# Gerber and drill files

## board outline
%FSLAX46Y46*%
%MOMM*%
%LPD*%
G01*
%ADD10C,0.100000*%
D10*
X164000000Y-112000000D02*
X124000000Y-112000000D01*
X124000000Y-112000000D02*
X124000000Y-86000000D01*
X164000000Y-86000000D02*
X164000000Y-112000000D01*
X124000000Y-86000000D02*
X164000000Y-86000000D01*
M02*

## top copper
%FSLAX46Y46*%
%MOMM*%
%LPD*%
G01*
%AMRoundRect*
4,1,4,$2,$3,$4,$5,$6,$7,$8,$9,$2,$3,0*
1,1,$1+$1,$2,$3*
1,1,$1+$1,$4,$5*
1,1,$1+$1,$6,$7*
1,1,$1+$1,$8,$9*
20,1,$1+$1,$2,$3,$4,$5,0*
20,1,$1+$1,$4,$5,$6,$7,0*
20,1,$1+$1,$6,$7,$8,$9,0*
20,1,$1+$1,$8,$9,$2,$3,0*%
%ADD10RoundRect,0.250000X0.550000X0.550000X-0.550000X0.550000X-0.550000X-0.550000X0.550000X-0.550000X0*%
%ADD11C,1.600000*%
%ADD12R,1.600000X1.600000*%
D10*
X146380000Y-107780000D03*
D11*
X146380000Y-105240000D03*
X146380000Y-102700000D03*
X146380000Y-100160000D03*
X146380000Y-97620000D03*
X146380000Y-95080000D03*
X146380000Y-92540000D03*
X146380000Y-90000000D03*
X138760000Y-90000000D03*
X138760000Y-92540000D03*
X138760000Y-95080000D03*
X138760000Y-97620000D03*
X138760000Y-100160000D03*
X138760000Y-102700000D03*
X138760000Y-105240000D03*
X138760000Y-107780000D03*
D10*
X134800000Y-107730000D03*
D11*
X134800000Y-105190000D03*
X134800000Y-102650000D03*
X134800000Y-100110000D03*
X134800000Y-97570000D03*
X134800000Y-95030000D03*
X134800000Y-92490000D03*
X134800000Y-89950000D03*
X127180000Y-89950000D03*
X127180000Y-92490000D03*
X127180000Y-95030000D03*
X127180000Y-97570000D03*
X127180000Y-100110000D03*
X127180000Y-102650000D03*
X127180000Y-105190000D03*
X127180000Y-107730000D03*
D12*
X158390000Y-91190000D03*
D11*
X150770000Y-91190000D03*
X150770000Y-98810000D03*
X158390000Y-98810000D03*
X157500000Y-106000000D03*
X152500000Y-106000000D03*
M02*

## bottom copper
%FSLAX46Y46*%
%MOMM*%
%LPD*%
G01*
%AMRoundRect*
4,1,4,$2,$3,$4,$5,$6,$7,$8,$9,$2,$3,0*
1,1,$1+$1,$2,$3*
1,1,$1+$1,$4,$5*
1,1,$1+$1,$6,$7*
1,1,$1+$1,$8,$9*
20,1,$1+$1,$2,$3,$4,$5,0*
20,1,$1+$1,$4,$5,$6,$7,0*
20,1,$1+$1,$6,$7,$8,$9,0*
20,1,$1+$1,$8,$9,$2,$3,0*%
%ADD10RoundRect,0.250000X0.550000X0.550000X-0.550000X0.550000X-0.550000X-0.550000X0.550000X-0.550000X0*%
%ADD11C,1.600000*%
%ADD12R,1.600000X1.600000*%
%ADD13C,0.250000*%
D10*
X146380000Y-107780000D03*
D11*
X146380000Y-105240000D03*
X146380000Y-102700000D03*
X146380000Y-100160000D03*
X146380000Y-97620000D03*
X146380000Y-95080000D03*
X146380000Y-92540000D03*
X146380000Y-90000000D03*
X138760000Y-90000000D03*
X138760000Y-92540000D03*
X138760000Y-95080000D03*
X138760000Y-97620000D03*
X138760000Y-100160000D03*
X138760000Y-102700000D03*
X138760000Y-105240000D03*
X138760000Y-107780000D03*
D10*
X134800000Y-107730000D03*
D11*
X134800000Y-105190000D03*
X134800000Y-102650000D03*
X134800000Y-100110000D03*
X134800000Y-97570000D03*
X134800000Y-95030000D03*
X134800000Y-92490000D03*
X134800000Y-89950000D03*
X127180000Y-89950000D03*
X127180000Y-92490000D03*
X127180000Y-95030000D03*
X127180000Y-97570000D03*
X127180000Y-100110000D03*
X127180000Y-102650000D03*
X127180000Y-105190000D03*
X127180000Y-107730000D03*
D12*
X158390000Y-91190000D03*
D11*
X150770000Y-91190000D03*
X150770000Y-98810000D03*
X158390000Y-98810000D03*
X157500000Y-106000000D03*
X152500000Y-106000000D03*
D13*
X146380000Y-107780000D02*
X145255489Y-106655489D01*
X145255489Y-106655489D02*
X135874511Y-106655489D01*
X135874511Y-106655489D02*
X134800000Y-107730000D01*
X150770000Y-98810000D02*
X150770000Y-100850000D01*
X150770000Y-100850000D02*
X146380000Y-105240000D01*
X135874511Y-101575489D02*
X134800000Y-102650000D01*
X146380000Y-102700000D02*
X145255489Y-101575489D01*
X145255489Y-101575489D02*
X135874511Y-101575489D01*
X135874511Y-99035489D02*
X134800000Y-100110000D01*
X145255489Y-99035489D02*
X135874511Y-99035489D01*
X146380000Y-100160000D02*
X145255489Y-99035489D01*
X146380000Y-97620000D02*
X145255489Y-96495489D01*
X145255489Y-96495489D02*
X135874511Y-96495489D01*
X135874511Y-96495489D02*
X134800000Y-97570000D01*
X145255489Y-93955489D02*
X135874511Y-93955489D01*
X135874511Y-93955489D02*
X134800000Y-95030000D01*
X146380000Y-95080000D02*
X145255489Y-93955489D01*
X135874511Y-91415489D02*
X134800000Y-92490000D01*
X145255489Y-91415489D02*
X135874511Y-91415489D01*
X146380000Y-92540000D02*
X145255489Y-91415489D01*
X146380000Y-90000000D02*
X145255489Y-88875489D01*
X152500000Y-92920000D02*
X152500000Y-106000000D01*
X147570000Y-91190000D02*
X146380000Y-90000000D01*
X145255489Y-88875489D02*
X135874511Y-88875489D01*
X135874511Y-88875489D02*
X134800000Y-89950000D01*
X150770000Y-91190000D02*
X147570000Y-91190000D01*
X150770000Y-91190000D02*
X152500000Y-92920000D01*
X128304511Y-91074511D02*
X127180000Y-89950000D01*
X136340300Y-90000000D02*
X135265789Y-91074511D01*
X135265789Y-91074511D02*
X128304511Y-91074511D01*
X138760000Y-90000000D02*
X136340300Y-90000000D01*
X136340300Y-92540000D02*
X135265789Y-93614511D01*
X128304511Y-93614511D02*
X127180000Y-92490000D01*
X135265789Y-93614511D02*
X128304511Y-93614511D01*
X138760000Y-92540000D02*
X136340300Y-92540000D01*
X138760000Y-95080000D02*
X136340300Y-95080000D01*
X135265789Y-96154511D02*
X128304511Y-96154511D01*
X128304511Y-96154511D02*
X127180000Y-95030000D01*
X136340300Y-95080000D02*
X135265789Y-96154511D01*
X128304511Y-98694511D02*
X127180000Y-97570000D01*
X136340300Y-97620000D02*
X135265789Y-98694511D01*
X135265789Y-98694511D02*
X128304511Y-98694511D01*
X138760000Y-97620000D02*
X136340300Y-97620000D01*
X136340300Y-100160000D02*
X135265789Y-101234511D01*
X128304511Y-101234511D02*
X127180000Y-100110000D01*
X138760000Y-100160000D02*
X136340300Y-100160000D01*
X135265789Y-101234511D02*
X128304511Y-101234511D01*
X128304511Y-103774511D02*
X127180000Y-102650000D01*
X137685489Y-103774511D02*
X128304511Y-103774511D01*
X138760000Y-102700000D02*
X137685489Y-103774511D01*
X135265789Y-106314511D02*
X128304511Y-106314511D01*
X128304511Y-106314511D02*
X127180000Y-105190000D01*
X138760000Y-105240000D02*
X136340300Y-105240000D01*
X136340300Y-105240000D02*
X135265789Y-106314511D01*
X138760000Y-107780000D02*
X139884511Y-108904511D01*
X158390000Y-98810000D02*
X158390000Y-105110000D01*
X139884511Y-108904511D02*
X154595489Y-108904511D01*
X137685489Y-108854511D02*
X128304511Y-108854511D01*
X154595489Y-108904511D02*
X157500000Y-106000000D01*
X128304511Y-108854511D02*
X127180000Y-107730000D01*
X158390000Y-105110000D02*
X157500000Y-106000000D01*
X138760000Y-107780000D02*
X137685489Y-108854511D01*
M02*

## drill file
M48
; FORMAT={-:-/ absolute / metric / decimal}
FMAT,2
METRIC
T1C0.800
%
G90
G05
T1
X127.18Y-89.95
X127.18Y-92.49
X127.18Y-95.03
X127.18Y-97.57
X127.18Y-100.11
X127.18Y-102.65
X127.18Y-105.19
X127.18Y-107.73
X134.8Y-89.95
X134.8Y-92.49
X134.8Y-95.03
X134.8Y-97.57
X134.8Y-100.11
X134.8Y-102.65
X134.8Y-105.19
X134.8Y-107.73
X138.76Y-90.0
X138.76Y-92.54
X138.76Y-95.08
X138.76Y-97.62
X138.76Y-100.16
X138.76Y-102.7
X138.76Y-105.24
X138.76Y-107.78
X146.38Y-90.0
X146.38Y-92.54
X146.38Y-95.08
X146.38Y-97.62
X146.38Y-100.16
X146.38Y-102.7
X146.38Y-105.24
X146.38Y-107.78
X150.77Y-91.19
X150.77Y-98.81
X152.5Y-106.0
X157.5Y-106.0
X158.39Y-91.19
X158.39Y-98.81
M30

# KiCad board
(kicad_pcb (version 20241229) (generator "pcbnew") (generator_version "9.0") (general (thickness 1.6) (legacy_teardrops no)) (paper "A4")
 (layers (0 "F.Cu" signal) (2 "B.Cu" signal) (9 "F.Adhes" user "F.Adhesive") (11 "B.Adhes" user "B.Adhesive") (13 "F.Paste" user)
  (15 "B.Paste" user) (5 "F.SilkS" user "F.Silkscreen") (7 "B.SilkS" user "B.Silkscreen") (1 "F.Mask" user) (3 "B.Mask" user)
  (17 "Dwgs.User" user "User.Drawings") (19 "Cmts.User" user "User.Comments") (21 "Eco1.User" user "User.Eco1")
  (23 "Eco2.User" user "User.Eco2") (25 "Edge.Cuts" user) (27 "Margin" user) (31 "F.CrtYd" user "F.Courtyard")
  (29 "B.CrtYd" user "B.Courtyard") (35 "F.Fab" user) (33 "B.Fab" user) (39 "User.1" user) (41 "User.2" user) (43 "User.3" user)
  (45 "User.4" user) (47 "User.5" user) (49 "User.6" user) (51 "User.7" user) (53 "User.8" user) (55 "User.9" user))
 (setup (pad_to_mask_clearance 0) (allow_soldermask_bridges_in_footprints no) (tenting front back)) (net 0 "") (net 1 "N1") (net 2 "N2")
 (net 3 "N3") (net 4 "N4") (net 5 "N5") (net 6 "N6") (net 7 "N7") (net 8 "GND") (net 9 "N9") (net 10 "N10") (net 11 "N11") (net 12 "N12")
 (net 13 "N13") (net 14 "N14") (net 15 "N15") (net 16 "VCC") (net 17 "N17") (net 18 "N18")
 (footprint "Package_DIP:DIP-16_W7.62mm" (layer "F.Cu") (at 146.38 107.78 180)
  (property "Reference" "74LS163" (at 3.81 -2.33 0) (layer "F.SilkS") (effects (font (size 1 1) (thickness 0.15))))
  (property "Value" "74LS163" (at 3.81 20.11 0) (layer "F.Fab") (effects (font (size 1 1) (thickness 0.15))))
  (pad "1" thru_hole roundrect (at 0 0 180) (size 1.6 1.6) (drill 0.8) (layers "*.Cu" "*.Mask") (remove_unused_layers no)
   (roundrect_rratio 0.15625) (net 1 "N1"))
  (pad "2" thru_hole circle (at 0 2.54 180) (size 1.6 1.6) (drill 0.8) (layers "*.Cu" "*.Mask") (remove_unused_layers no) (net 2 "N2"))
  (pad "3" thru_hole circle (at 0 5.08 180) (size 1.6 1.6) (drill 0.8) (layers "*.Cu" "*.Mask") (remove_unused_layers no) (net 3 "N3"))
  (pad "4" thru_hole circle (at 0 7.62 180) (size 1.6 1.6) (drill 0.8) (layers "*.Cu" "*.Mask") (remove_unused_layers no) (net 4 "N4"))
  (pad "5" thru_hole circle (at 0 10.16 180) (size 1.6 1.6) (drill 0.8) (layers "*.Cu" "*.Mask") (remove_unused_layers no) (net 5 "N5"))
  (pad "6" thru_hole circle (at 0 12.7 180) (size 1.6 1.6) (drill 0.8) (layers "*.Cu" "*.Mask") (remove_unused_layers no) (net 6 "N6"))
  (pad "7" thru_hole circle (at 0 15.24 180) (size 1.6 1.6) (drill 0.8) (layers "*.Cu" "*.Mask") (remove_unused_layers no) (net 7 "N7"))
  (pad "8" thru_hole circle (at 0 17.78 180) (size 1.6 1.6) (drill 0.8) (layers "*.Cu" "*.Mask") (remove_unused_layers no) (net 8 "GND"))
  (pad "9" thru_hole circle (at 7.62 17.78 180) (size 1.6 1.6) (drill 0.8) (layers "*.Cu" "*.Mask") (remove_unused_layers no) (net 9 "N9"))
  (pad "10" thru_hole circle (at 7.62 15.24 180) (size 1.6 1.6) (drill 0.8) (layers "*.Cu" "*.Mask") (remove_unused_layers no)
   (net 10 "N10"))
  (pad "11" thru_hole circle (at 7.62 12.7 180) (size 1.6 1.6) (drill 0.8) (layers "*.Cu" "*.Mask") (remove_unused_layers no) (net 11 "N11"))
  (pad "12" thru_hole circle (at 7.62 10.16 180) (size 1.6 1.6) (drill 0.8) (layers "*.Cu" "*.Mask") (remove_unused_layers no)
   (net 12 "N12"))
  (pad "13" thru_hole circle (at 7.62 7.62 180) (size 1.6 1.6) (drill 0.8) (layers "*.Cu" "*.Mask") (remove_unused_layers no) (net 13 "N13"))
  (pad "14" thru_hole circle (at 7.62 5.08 180) (size 1.6 1.6) (drill 0.8) (layers "*.Cu" "*.Mask") (remove_unused_layers no) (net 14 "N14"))
  (pad "15" thru_hole circle (at 7.62 2.54 180) (size 1.6 1.6) (drill 0.8) (layers "*.Cu" "*.Mask") (remove_unused_layers no) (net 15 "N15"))
  (pad "16" thru_hole circle (at 7.62 0 180) (size 1.6 1.6) (drill 0.8) (layers "*.Cu" "*.Mask") (remove_unused_layers no) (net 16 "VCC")))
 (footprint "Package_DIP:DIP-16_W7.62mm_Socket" (layer "F.Cu") (at 134.8 107.73 180)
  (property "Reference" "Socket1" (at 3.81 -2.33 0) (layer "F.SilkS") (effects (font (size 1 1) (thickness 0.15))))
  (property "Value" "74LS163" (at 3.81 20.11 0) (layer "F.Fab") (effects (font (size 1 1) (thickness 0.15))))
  (pad "1" thru_hole roundrect (at 0 0 180) (size 1.6 1.6) (drill 0.8) (layers "*.Cu" "*.Mask") (remove_unused_layers no)
   (roundrect_rratio 0.15625) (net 1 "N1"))
  (pad "2" thru_hole circle (at 0 2.54 180) (size 1.6 1.6) (drill 0.8) (layers "*.Cu" "*.Mask") (remove_unused_layers no) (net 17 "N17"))
  (pad "3" thru_hole circle (at 0 5.08 180) (size 1.6 1.6) (drill 0.8) (layers "*.Cu" "*.Mask") (remove_unused_layers no) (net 3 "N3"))
  (pad "4" thru_hole circle (at 0 7.62 180) (size 1.6 1.6) (drill 0.8) (layers "*.Cu" "*.Mask") (remove_unused_layers no) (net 4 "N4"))
  (pad "5" thru_hole circle (at 0 10.16 180) (size 1.6 1.6) (drill 0.8) (layers "*.Cu" "*.Mask") (remove_unused_layers no) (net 5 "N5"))
  (pad "6" thru_hole circle (at 0 12.7 180) (size 1.6 1.6) (drill 0.8) (layers "*.Cu" "*.Mask") (remove_unused_layers no) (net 6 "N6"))
  (pad "7" thru_hole circle (at 0 15.24 180) (size 1.6 1.6) (drill 0.8) (layers "*.Cu" "*.Mask") (remove_unused_layers no) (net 7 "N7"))
  (pad "8" thru_hole circle (at 0 17.78 180) (size 1.6 1.6) (drill 0.8) (layers "*.Cu" "*.Mask") (remove_unused_layers no) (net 8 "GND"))
  (pad "9" thru_hole circle (at 7.62 17.78 180) (size 1.6 1.6) (drill 0.8) (layers "*.Cu" "*.Mask") (remove_unused_layers no) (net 9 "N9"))
  (pad "10" thru_hole circle (at 7.62 15.24 180) (size 1.6 1.6) (drill 0.8) (layers "*.Cu" "*.Mask") (remove_unused_layers no)
   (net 10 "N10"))
  (pad "11" thru_hole circle (at 7.62 12.7 180) (size 1.6 1.6) (drill 0.8) (layers "*.Cu" "*.Mask") (remove_unused_layers no) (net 11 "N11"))
  (pad "12" thru_hole circle (at 7.62 10.16 180) (size 1.6 1.6) (drill 0.8) (layers "*.Cu" "*.Mask") (remove_unused_layers no)
   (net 12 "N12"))
  (pad "13" thru_hole circle (at 7.62 7.62 180) (size 1.6 1.6) (drill 0.8) (layers "*.Cu" "*.Mask") (remove_unused_layers no) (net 13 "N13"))
  (pad "14" thru_hole circle (at 7.62 5.08 180) (size 1.6 1.6) (drill 0.8) (layers "*.Cu" "*.Mask") (remove_unused_layers no) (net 14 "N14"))
  (pad "15" thru_hole circle (at 7.62 2.54 180) (size 1.6 1.6) (drill 0.8) (layers "*.Cu" "*.Mask") (remove_unused_layers no) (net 15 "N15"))
  (pad "16" thru_hole circle (at 7.62 0 180) (size 1.6 1.6) (drill 0.8) (layers "*.Cu" "*.Mask") (remove_unused_layers no) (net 16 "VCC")))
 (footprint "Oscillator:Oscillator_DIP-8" (layer "F.Cu") (at 158.39 91.19 180)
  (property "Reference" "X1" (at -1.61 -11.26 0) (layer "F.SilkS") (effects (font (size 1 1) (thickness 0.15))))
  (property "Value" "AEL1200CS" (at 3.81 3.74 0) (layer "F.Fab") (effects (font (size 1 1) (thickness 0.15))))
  (pad "1" thru_hole rect (at 0 0 180) (size 1.6 1.6) (drill 0.8) (layers "*.Cu" "*.Mask") (remove_unused_layers no) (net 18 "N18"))
  (pad "4" thru_hole circle (at 7.62 0 180) (size 1.6 1.6) (drill 0.8) (layers "*.Cu" "*.Mask") (remove_unused_layers no) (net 8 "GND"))
  (pad "5" thru_hole circle (at 7.62 -7.62 180) (size 1.6 1.6) (drill 0.8) (layers "*.Cu" "*.Mask") (remove_unused_layers no) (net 2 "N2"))
  (pad "8" thru_hole circle (at 0 -7.62 180) (size 1.6 1.6) (drill 0.8) (layers "*.Cu" "*.Mask") (remove_unused_layers no) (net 16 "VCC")))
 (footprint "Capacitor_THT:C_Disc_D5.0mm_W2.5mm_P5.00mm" (layer "F.Cu") (at 157.5 106 180)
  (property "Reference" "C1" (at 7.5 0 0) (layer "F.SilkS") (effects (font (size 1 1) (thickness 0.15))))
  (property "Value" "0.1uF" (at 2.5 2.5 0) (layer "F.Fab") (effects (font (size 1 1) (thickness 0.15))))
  (pad "1" thru_hole circle (at 0 0 180) (size 1.6 1.6) (drill 0.8) (layers "*.Cu" "*.Mask") (remove_unused_layers no) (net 16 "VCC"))
  (pad "2" thru_hole circle (at 5 0 180) (size 1.6 1.6) (drill 0.8) (layers "*.Cu" "*.Mask") (remove_unused_layers no) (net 8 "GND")))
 (gr_line (start 164 112) (end 124 112) (stroke (width 0.1) (type solid)) (layer "Edge.Cuts"))
 (gr_line (start 124 112) (end 124 86) (stroke (width 0.1) (type solid)) (layer "Edge.Cuts"))
 (gr_line (start 164 86) (end 164 112) (stroke (width 0.1) (type solid)) (layer "Edge.Cuts"))
 (gr_line (start 124 86) (end 164 86) (stroke (width 0.1) (type solid)) (layer "Edge.Cuts"))
 (segment (start 146.38 107.78) (end 145.255489 106.655489) (width 0.25) (layer "B.Cu") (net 1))
 (segment (start 145.255489 106.655489) (end 135.874511 106.655489) (width 0.25) (layer "B.Cu") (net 1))
 (segment (start 135.874511 106.655489) (end 134.8 107.73) (width 0.25) (layer "B.Cu") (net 1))
 (segment (start 150.77 98.81) (end 150.77 100.85) (width 0.25) (layer "B.Cu") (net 2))
 (segment (start 150.77 100.85) (end 146.38 105.24) (width 0.25) (layer "B.Cu") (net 2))
 (segment (start 135.874511 101.575489) (end 134.8 102.65) (width 0.25) (layer "B.Cu") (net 3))
 (segment (start 146.38 102.7) (end 145.255489 101.575489) (width 0.25) (layer "B.Cu") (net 3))
 (segment (start 145.255489 101.575489) (end 135.874511 101.575489) (width 0.25) (layer "B.Cu") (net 3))
 (segment (start 135.874511 99.035489) (end 134.8 100.11) (width 0.25) (layer "B.Cu") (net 4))
 (segment (start 145.255489 99.035489) (end 135.874511 99.035489) (width 0.25) (layer "B.Cu") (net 4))
 (segment (start 146.38 100.16) (end 145.255489 99.035489) (width 0.25) (layer "B.Cu") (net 4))
 (segment (start 146.38 97.62) (end 145.255489 96.495489) (width 0.25) (layer "B.Cu") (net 5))
 (segment (start 145.255489 96.495489) (end 135.874511 96.495489) (width 0.25) (layer "B.Cu") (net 5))
 (segment (start 135.874511 96.495489) (end 134.8 97.57) (width 0.25) (layer "B.Cu") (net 5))
 (segment (start 145.255489 93.955489) (end 135.874511 93.955489) (width 0.25) (layer "B.Cu") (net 6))
 (segment (start 135.874511 93.955489) (end 134.8 95.03) (width 0.25) (layer "B.Cu") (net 6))
 (segment (start 146.38 95.08) (end 145.255489 93.955489) (width 0.25) (layer "B.Cu") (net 6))
 (segment (start 135.874511 91.415489) (end 134.8 92.49) (width 0.25) (layer "B.Cu") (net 7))
 (segment (start 145.255489 91.415489) (end 135.874511 91.415489) (width 0.25) (layer "B.Cu") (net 7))
 (segment (start 146.38 92.54) (end 145.255489 91.415489) (width 0.25) (layer "B.Cu") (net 7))
 (segment (start 146.38 90) (end 145.255489 88.875489) (width 0.25) (layer "B.Cu") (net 8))
 (segment (start 152.5 92.92) (end 152.5 106) (width 0.25) (layer "B.Cu") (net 8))
 (segment (start 147.57 91.19) (end 146.38 90) (width 0.25) (layer "B.Cu") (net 8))
 (segment (start 145.255489 88.875489) (end 135.874511 88.875489) (width 0.25) (layer "B.Cu") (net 8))
 (segment (start 135.874511 88.875489) (end 134.8 89.95) (width 0.25) (layer "B.Cu") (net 8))
 (segment (start 150.77 91.19) (end 147.57 91.19) (width 0.25) (layer "B.Cu") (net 8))
 (segment (start 150.77 91.19) (end 152.5 92.92) (width 0.25) (layer "B.Cu") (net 8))
 (segment (start 128.304511 91.074511) (end 127.18 89.95) (width 0.25) (layer "B.Cu") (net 9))
 (segment (start 136.3403 90) (end 135.265789 91.074511) (width 0.25) (layer "B.Cu") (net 9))
 (segment (start 135.265789 91.074511) (end 128.304511 91.074511) (width 0.25) (layer "B.Cu") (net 9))
 (segment (start 138.76 90) (end 136.3403 90) (width 0.25) (layer "B.Cu") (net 9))
 (segment (start 136.3403 92.54) (end 135.265789 93.614511) (width 0.25) (layer "B.Cu") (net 10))
 (segment (start 128.304511 93.614511) (end 127.18 92.49) (width 0.25) (layer "B.Cu") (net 10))
 (segment (start 135.265789 93.614511) (end 128.304511 93.614511) (width 0.25) (layer "B.Cu") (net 10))
 (segment (start 138.76 92.54) (end 136.3403 92.54) (width 0.25) (layer "B.Cu") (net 10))
 (segment (start 138.76 95.08) (end 136.3403 95.08) (width 0.25) (layer "B.Cu") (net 11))
 (segment (start 135.265789 96.154511) (end 128.304511 96.154511) (width 0.25) (layer "B.Cu") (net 11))
 (segment (start 128.304511 96.154511) (end 127.18 95.03) (width 0.25) (layer "B.Cu") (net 11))
 (segment (start 136.3403 95.08) (end 135.265789 96.154511) (width 0.25) (layer "B.Cu") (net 11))
 (segment (start 128.304511 98.694511) (end 127.18 97.57) (width 0.25) (layer "B.Cu") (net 12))
 (segment (start 136.3403 97.62) (end 135.265789 98.694511) (width 0.25) (layer "B.Cu") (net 12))
 (segment (start 135.265789 98.694511) (end 128.304511 98.694511) (width 0.25) (layer "B.Cu") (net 12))
 (segment (start 138.76 97.62) (end 136.3403 97.62) (width 0.25) (layer "B.Cu") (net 12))
 (segment (start 136.3403 100.16) (end 135.265789 101.234511) (width 0.25) (layer "B.Cu") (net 13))
 (segment (start 128.304511 101.234511) (end 127.18 100.11) (width 0.25) (layer "B.Cu") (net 13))
 (segment (start 138.76 100.16) (end 136.3403 100.16) (width 0.25) (layer "B.Cu") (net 13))
 (segment (start 135.265789 101.234511) (end 128.304511 101.234511) (width 0.25) (layer "B.Cu") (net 13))
 (segment (start 128.304511 103.774511) (end 127.18 102.65) (width 0.25) (layer "B.Cu") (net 14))
 (segment (start 137.685489 103.774511) (end 128.304511 103.774511) (width 0.25) (layer "B.Cu") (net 14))
 (segment (start 138.76 102.7) (end 137.685489 103.774511) (width 0.25) (layer "B.Cu") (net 14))
 (segment (start 135.265789 106.314511) (end 128.304511 106.314511) (width 0.25) (layer "B.Cu") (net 15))
 (segment (start 128.304511 106.314511) (end 127.18 105.19) (width 0.25) (layer "B.Cu") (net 15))
 (segment (start 138.76 105.24) (end 136.3403 105.24) (width 0.25) (layer "B.Cu") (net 15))
 (segment (start 136.3403 105.24) (end 135.265789 106.314511) (width 0.25) (layer "B.Cu") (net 15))
 (segment (start 138.76 107.78) (end 139.884511 108.904511) (width 0.25) (layer "B.Cu") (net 16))
 (segment (start 158.39 98.81) (end 158.39 105.11) (width 0.25) (layer "B.Cu") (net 16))
 (segment (start 139.884511 108.904511) (end 154.595489 108.904511) (width 0.25) (layer "B.Cu") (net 16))
 (segment (start 137.685489 108.854511) (end 128.304511 108.854511) (width 0.25) (layer "B.Cu") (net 16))
 (segment (start 154.595489 108.904511) (end 157.5 106) (width 0.25) (layer "B.Cu") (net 16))
 (segment (start 128.304511 108.854511) (end 127.18 107.73) (width 0.25) (layer "B.Cu") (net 16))
 (segment (start 158.39 105.11) (end 157.5 106) (width 0.25) (layer "B.Cu") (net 16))
 (segment (start 138.76 107.78) (end 137.685489 108.854511) (width 0.25) (layer "B.Cu") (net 16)))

